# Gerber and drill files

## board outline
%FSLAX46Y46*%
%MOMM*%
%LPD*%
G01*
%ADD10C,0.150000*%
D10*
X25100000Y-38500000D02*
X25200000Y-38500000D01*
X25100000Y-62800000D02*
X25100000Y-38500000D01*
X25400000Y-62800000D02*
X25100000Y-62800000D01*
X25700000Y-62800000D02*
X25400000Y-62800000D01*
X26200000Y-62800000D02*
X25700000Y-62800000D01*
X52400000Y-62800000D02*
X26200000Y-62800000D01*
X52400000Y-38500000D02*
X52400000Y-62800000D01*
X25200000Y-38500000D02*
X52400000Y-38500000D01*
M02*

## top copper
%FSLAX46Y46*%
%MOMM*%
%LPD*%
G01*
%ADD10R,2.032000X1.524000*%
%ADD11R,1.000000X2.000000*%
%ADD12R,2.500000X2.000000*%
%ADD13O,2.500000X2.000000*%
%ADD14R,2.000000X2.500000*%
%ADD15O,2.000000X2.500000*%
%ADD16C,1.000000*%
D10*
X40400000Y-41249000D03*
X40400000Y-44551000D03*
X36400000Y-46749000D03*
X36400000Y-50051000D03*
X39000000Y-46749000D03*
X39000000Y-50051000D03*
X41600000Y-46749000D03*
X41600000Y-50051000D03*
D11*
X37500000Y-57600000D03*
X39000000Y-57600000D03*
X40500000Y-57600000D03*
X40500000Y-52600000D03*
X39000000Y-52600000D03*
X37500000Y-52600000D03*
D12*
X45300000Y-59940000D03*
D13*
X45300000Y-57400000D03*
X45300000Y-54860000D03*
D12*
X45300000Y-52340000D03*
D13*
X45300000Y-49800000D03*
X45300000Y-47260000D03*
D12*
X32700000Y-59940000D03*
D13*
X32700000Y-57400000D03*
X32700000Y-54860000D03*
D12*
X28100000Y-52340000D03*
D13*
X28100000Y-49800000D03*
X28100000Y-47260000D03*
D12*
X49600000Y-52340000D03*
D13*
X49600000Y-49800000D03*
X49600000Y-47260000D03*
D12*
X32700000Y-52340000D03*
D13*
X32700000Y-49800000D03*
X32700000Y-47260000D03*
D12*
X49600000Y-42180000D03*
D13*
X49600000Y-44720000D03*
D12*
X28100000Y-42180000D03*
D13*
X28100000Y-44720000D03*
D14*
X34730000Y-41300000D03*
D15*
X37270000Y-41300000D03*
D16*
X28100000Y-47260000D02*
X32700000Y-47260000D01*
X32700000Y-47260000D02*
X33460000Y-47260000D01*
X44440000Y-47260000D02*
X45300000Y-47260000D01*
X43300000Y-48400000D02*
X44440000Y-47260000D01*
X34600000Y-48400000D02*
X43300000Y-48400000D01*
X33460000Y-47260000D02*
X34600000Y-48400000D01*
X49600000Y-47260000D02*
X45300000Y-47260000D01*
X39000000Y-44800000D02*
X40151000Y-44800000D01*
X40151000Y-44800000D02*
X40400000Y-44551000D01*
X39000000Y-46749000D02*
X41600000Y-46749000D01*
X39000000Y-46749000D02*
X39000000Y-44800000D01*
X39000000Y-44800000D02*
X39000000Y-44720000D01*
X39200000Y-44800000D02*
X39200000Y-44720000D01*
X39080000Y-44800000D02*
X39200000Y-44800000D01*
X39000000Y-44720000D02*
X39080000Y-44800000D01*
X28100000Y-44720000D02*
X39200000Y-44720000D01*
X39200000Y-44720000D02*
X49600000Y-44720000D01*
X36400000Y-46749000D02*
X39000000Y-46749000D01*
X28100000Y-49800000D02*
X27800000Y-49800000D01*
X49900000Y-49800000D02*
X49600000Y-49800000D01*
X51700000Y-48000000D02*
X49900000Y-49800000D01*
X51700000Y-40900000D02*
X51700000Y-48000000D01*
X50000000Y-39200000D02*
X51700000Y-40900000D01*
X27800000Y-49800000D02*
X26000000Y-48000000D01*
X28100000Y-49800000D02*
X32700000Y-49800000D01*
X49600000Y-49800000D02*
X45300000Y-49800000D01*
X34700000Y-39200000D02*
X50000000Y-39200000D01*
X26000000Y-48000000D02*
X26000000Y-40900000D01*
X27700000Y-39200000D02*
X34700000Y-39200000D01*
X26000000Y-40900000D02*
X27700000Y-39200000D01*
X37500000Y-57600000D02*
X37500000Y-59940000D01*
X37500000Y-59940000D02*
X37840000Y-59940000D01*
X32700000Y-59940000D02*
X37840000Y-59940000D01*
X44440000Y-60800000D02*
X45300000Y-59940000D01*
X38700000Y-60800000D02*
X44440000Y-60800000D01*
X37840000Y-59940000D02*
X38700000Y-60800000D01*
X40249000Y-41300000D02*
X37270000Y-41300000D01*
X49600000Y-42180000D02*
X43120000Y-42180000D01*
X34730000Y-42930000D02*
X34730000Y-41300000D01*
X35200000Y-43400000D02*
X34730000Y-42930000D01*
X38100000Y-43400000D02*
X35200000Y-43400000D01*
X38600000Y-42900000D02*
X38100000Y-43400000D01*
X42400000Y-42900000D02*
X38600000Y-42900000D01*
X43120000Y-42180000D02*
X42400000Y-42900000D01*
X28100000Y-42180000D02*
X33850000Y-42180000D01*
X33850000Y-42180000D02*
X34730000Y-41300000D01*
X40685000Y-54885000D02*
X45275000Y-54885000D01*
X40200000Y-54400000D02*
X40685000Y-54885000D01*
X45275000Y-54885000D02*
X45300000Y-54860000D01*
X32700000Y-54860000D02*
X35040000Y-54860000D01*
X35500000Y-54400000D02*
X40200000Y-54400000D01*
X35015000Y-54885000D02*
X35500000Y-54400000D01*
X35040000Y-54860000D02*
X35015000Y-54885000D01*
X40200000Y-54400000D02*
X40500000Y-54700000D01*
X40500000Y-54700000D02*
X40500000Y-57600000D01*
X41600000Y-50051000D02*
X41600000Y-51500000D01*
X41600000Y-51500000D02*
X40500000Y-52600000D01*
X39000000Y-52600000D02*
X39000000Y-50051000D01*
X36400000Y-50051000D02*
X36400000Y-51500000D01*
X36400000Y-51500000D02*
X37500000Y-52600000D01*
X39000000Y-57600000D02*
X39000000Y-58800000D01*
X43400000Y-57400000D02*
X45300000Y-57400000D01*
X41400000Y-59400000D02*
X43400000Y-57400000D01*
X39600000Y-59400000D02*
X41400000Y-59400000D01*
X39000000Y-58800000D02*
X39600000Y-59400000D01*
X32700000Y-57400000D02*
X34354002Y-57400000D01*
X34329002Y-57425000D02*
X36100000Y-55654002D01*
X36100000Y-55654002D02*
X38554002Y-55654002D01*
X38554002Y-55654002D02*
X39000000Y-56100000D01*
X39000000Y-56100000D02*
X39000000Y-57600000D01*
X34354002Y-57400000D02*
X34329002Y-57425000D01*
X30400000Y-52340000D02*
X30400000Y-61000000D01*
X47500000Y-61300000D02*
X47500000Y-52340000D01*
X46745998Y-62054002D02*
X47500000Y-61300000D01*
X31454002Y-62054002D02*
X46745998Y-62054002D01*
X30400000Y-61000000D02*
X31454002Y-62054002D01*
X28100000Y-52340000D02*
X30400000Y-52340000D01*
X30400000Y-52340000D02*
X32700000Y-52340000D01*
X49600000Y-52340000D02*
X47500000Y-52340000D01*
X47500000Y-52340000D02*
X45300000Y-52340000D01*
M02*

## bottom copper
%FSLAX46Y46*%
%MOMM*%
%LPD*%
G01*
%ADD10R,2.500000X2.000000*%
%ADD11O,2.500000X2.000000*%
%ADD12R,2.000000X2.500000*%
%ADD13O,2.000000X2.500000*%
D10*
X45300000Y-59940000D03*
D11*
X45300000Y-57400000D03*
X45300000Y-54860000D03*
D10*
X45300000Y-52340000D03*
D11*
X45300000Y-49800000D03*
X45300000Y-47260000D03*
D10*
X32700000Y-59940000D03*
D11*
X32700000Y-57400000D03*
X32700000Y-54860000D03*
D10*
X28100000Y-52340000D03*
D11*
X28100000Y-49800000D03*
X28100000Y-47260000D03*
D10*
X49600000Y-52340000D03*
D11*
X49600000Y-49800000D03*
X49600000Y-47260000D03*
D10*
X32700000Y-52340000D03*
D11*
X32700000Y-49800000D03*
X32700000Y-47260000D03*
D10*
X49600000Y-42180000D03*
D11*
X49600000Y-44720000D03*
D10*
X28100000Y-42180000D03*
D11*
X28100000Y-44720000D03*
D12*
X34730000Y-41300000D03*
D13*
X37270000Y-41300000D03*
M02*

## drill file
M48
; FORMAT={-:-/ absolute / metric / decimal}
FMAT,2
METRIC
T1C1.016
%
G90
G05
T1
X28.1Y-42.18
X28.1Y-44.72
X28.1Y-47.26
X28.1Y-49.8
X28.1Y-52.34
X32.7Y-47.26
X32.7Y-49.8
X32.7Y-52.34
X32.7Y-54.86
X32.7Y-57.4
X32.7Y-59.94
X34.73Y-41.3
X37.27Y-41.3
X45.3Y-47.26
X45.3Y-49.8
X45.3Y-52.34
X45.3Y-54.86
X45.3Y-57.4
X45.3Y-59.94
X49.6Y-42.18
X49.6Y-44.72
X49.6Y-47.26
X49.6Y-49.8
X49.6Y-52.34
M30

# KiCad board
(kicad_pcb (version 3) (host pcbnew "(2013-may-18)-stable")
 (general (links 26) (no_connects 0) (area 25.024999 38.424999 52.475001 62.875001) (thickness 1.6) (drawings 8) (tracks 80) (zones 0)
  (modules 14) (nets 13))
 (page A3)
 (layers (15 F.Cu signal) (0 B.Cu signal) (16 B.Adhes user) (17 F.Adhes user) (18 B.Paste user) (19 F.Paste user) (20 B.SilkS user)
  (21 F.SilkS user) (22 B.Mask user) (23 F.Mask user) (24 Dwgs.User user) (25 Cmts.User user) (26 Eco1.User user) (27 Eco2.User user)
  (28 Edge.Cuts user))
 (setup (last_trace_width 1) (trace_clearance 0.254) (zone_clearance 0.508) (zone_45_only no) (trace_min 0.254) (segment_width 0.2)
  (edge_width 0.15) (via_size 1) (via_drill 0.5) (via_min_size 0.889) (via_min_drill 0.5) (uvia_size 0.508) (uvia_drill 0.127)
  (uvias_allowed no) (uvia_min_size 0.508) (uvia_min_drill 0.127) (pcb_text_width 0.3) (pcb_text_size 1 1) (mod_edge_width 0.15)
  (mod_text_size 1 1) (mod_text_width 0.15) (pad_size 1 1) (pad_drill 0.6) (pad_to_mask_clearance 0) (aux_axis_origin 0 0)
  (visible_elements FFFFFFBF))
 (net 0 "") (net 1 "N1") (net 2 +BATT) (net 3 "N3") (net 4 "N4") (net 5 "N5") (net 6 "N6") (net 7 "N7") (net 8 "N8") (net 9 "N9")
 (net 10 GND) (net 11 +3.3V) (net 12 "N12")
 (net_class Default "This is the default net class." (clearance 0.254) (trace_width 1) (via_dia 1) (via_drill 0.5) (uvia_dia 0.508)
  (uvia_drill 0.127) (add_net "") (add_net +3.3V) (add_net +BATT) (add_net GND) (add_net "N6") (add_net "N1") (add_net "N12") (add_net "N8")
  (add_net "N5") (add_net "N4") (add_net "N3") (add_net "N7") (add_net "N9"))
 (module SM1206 (layer F.Cu) (at 40.4 42.9 270)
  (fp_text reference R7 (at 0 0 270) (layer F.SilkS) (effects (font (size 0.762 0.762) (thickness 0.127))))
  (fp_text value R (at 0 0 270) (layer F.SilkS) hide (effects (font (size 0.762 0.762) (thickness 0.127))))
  (pad 1 smd rect (at -1.651 0 270) (size 1.524 2.032) (layers F.Cu F.Paste F.Mask) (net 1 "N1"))
  (pad 2 smd rect (at 1.651 0 270) (size 1.524 2.032) (layers F.Cu F.Paste F.Mask) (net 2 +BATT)))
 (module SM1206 (layer F.Cu) (at 36.4 48.4 270)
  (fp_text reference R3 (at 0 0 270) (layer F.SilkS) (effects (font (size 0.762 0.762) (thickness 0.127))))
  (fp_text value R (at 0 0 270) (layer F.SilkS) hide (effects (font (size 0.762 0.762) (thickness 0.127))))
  (pad 1 smd rect (at -1.651 0 270) (size 1.524 2.032) (layers F.Cu F.Paste F.Mask) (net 2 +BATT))
  (pad 2 smd rect (at 1.651 0 270) (size 1.524 2.032) (layers F.Cu F.Paste F.Mask) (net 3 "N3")))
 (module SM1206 (layer F.Cu) (at 39 48.4 270)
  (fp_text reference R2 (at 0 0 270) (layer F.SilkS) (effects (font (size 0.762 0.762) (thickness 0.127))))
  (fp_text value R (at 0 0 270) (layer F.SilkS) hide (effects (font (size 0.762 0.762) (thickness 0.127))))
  (pad 1 smd rect (at -1.651 0 270) (size 1.524 2.032) (layers F.Cu F.Paste F.Mask) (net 2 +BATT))
  (pad 2 smd rect (at 1.651 0 270) (size 1.524 2.032) (layers F.Cu F.Paste F.Mask) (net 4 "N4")))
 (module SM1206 (layer F.Cu) (at 41.6 48.4 270)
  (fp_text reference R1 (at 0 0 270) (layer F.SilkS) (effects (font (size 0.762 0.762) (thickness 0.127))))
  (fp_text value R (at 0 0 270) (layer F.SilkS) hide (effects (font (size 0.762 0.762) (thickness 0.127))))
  (pad 1 smd rect (at -1.651 0 270) (size 1.524 2.032) (layers F.Cu F.Paste F.Mask) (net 2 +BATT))
  (pad 2 smd rect (at 1.651 0 270) (size 1.524 2.032) (layers F.Cu F.Paste F.Mask) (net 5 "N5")))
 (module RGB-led (layer F.Cu) (at 39 55.1 270)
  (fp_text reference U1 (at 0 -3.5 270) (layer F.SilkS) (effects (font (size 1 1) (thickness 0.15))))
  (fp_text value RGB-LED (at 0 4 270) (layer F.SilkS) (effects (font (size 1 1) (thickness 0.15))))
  (pad 1 smd rect (at 2.5 1.5 270) (size 2 1) (layers F.Cu F.Paste F.Mask) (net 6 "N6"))
  (pad 2 smd rect (at 2.5 0 270) (size 2 1) (layers F.Cu F.Paste F.Mask) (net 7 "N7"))
  (pad 3 smd rect (at 2.5 -1.5 270) (size 2 1) (layers F.Cu F.Paste F.Mask) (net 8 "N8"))
  (pad 4 smd rect (at -2.5 -1.5 270) (size 2 1) (layers F.Cu F.Paste F.Mask) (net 5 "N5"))
  (pad 5 smd rect (at -2.5 0 270) (size 2 1) (layers F.Cu F.Paste F.Mask) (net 4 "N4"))
  (pad 6 smd rect (at -2.5 1.5 270) (size 2 1) (layers F.Cu F.Paste F.Mask) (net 3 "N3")))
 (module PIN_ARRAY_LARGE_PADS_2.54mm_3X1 (layer F.Cu) (at 45.3 57.4 90)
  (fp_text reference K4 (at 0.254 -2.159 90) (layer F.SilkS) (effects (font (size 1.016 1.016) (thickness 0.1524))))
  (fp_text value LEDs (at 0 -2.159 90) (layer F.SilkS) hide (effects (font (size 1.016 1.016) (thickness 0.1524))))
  (pad 1 thru_hole rect (at -2.54 0 90) (size 2 2.5) (drill 1.016) (layers *.Cu *.Mask F.SilkS) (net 6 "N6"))
  (pad 2 thru_hole oval (at 0 0 90) (size 2 2.5) (drill 1.016) (layers *.Cu *.Mask F.SilkS) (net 7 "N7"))
  (pad 3 thru_hole oval (at 2.54 0 90) (size 2 2.5) (drill 1.016) (layers *.Cu *.Mask F.SilkS) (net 8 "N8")))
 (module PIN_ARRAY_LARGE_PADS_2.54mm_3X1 (layer F.Cu) (at 45.3 49.8 90)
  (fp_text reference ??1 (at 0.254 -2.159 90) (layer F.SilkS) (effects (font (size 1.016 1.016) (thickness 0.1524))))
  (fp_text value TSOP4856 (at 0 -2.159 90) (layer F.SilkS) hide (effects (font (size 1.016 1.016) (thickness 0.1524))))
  (pad 1 thru_hole rect (at -2.54 0 90) (size 2 2.5) (drill 1.016) (layers *.Cu *.Mask F.SilkS) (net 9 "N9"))
  (pad 2 thru_hole oval (at 0 0 90) (size 2 2.5) (drill 1.016) (layers *.Cu *.Mask F.SilkS) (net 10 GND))
  (pad 3 thru_hole oval (at 2.54 0 90) (size 2 2.5) (drill 1.016) (layers *.Cu *.Mask F.SilkS) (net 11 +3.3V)))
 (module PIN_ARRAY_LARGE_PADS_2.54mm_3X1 (layer F.Cu) (at 32.7 57.4 90)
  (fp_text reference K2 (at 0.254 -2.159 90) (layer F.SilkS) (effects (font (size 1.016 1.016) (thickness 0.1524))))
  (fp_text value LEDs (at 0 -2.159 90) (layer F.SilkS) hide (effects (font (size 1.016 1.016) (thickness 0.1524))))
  (pad 1 thru_hole rect (at -2.54 0 90) (size 2 2.5) (drill 1.016) (layers *.Cu *.Mask F.SilkS) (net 6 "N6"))
  (pad 2 thru_hole oval (at 0 0 90) (size 2 2.5) (drill 1.016) (layers *.Cu *.Mask F.SilkS) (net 7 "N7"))
  (pad 3 thru_hole oval (at 2.54 0 90) (size 2 2.5) (drill 1.016) (layers *.Cu *.Mask F.SilkS) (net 8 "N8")))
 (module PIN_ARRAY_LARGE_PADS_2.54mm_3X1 (layer F.Cu) (at 28.1 49.8 90)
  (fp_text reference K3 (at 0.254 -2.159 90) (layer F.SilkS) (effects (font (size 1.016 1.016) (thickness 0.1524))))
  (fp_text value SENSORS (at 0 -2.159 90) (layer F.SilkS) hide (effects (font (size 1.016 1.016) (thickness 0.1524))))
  (pad 1 thru_hole rect (at -2.54 0 90) (size 2 2.5) (drill 1.016) (layers *.Cu *.Mask F.SilkS) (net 9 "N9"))
  (pad 2 thru_hole oval (at 0 0 90) (size 2 2.5) (drill 1.016) (layers *.Cu *.Mask F.SilkS) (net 10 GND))
  (pad 3 thru_hole oval (at 2.54 0 90) (size 2 2.5) (drill 1.016) (layers *.Cu *.Mask F.SilkS) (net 11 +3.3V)))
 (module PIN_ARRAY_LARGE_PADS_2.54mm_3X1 (layer F.Cu) (at 49.6 49.8 90)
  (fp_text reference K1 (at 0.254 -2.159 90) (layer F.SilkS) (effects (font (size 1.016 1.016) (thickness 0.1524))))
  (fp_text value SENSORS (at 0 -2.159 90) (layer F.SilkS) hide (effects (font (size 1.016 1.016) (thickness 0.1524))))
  (pad 1 thru_hole rect (at -2.54 0 90) (size 2 2.5) (drill 1.016) (layers *.Cu *.Mask F.SilkS) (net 9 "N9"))
  (pad 2 thru_hole oval (at 0 0 90) (size 2 2.5) (drill 1.016) (layers *.Cu *.Mask F.SilkS) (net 10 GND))
  (pad 3 thru_hole oval (at 2.54 0 90) (size 2 2.5) (drill 1.016) (layers *.Cu *.Mask F.SilkS) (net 11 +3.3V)))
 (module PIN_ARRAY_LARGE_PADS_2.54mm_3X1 (layer F.Cu) (at 32.7 49.8 90)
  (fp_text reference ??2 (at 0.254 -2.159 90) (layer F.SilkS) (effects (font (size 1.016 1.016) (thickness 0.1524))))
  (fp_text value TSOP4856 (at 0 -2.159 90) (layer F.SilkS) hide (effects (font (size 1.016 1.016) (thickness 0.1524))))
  (pad 1 thru_hole rect (at -2.54 0 90) (size 2 2.5) (drill 1.016) (layers *.Cu *.Mask F.SilkS) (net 9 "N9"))
  (pad 2 thru_hole oval (at 0 0 90) (size 2 2.5) (drill 1.016) (layers *.Cu *.Mask F.SilkS) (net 10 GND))
  (pad 3 thru_hole oval (at 2.54 0 90) (size 2 2.5) (drill 1.016) (layers *.Cu *.Mask F.SilkS) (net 11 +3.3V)))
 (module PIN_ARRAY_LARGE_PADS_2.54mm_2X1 (layer F.Cu) (at 49.6 43.45 270)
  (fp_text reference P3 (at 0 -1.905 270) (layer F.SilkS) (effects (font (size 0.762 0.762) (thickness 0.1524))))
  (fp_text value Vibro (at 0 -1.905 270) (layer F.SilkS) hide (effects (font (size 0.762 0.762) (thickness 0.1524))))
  (pad 1 thru_hole rect (at -1.27 0 270) (size 2 2.5) (drill 1.016) (layers *.Cu *.Mask F.SilkS) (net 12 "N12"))
  (pad 2 thru_hole oval (at 1.27 0 270) (size 2 2.5) (drill 1.016) (layers *.Cu *.Mask F.SilkS) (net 2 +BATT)))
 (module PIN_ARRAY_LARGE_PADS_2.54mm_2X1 (layer F.Cu) (at 28.1 43.45 270)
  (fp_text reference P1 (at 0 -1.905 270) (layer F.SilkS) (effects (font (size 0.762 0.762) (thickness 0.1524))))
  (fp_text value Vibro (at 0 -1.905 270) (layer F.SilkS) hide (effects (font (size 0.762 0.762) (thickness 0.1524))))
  (pad 1 thru_hole rect (at -1.27 0 270) (size 2 2.5) (drill 1.016) (layers *.Cu *.Mask F.SilkS) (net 12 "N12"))
  (pad 2 thru_hole oval (at 1.27 0 270) (size 2 2.5) (drill 1.016) (layers *.Cu *.Mask F.SilkS) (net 2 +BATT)))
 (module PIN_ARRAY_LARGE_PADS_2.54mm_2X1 (layer F.Cu) (at 36 41.3)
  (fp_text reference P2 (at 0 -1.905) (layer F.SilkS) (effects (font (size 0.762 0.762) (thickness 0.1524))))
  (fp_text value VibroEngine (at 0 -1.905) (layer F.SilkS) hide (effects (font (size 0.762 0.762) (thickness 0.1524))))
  (pad 1 thru_hole rect (at -1.27 0) (size 2 2.5) (drill 1.016) (layers *.Cu *.Mask F.SilkS) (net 12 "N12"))
  (pad 2 thru_hole oval (at 1.27 0) (size 2 2.5) (drill 1.016) (layers *.Cu *.Mask F.SilkS) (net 1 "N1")))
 (gr_line (start 25.1 38.5) (end 25.2 38.5) (angle 90) (layer Edge.Cuts) (width 0.15))
 (gr_line (start 25.1 62.8) (end 25.1 38.5) (angle 90) (layer Edge.Cuts) (width 0.15))
 (gr_line (start 25.4 62.8) (end 25.1 62.8) (angle 90) (layer Edge.Cuts) (width 0.15))
 (gr_line (start 25.7 62.8) (end 25.4 62.8) (angle 90) (layer Edge.Cuts) (width 0.15))
 (gr_line (start 26.2 62.8) (end 25.7 62.8) (angle 90) (layer Edge.Cuts) (width 0.15))
 (gr_line (start 52.4 62.8) (end 26.2 62.8) (angle 90) (layer Edge.Cuts) (width 0.15))
 (gr_line (start 52.4 38.5) (end 52.4 62.8) (angle 90) (layer Edge.Cuts) (width 0.15))
 (gr_line (start 25.2 38.5) (end 52.4 38.5) (angle 90) (layer Edge.Cuts) (width 0.15))
 (segment (start 28.1 47.26) (end 32.7 47.26) (width 1) (layer F.Cu) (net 11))
 (segment (start 32.7 47.26) (end 33.46 47.26) (width 1) (layer F.Cu) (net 11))
 (segment (start 44.44 47.26) (end 45.3 47.26) (width 1) (layer F.Cu) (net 11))
 (segment (start 43.3 48.4) (end 44.44 47.26) (width 1) (layer F.Cu) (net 11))
 (segment (start 34.6 48.4) (end 43.3 48.4) (width 1) (layer F.Cu) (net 11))
 (segment (start 33.46 47.26) (end 34.6 48.4) (width 1) (layer F.Cu) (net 11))
 (segment (start 49.6 47.26) (end 45.3 47.26) (width 1) (layer F.Cu) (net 11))
 (segment (start 39 44.8) (end 40.151 44.8) (width 1) (layer F.Cu) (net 2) (status 800000))
 (segment (start 40.151 44.8) (end 40.4 44.551) (width 1) (layer F.Cu) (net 2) (status C00000))
 (segment (start 39 46.749) (end 41.6 46.749) (width 1) (layer F.Cu) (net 2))
 (segment (start 39 46.749) (end 39 44.8) (width 1) (layer F.Cu) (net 2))
 (segment (start 39 44.8) (end 39 44.72) (width 1) (layer F.Cu) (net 2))
 (segment (start 39.2 44.8) (end 39.2 44.72) (width 1) (layer F.Cu) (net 2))
 (segment (start 39.08 44.8) (end 39.2 44.8) (width 1) (layer F.Cu) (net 2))
 (segment (start 39 44.72) (end 39.08 44.8) (width 1) (layer F.Cu) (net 2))
 (segment (start 28.1 44.72) (end 39.2 44.72) (width 1) (layer F.Cu) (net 2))
 (segment (start 39.2 44.72) (end 49.6 44.72) (width 1) (layer F.Cu) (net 2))
 (segment (start 36.4 46.749) (end 39 46.749) (width 1) (layer F.Cu) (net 2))
 (segment (start 28.1 49.8) (end 27.8 49.8) (width 1) (layer F.Cu) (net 10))
 (segment (start 49.9 49.8) (end 49.6 49.8) (width 1) (layer F.Cu) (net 10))
 (segment (start 51.7 48) (end 49.9 49.8) (width 1) (layer F.Cu) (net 10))
 (segment (start 51.7 40.9) (end 51.7 48) (width 1) (layer F.Cu) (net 10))
 (segment (start 50 39.2) (end 51.7 40.9) (width 1) (layer F.Cu) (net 10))
 (segment (start 27.8 49.8) (end 26 48) (width 1) (layer F.Cu) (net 10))
 (segment (start 28.1 49.8) (end 32.7 49.8) (width 1) (layer F.Cu) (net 10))
 (segment (start 49.6 49.8) (end 45.3 49.8) (width 1) (layer F.Cu) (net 10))
 (segment (start 34.7 39.2) (end 50 39.2) (width 1) (layer F.Cu) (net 10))
 (segment (start 26 48) (end 26 40.9) (width 1) (layer F.Cu) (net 10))
 (segment (start 27.7 39.2) (end 34.7 39.2) (width 1) (layer F.Cu) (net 10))
 (segment (start 26 40.9) (end 27.7 39.2) (width 1) (layer F.Cu) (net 10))
 (segment (start 37.5 57.6) (end 37.5 59.94) (width 1) (layer F.Cu) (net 6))
 (segment (start 37.5 59.94) (end 37.84 59.94) (width 1) (layer F.Cu) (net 6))
 (segment (start 32.7 59.94) (end 37.84 59.94) (width 1) (layer F.Cu) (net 6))
 (segment (start 44.44 60.8) (end 45.3 59.94) (width 1) (layer F.Cu) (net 6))
 (segment (start 38.7 60.8) (end 44.44 60.8) (width 1) (layer F.Cu) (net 6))
 (segment (start 37.84 59.94) (end 38.7 60.8) (width 1) (layer F.Cu) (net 6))
 (segment (start 40.249 41.3) (end 37.27 41.3) (width 1) (layer F.Cu) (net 1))
 (segment (start 49.6 42.18) (end 43.12 42.18) (width 1) (layer F.Cu) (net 12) (status 400000))
 (segment (start 34.73 42.93) (end 34.73 41.3) (width 1) (layer F.Cu) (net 12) (status 800000))
 (segment (start 35.2 43.4) (end 34.73 42.93) (width 1) (layer F.Cu) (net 12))
 (segment (start 38.1 43.4) (end 35.2 43.4) (width 1) (layer F.Cu) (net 12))
 (segment (start 38.6 42.9) (end 38.1 43.4) (width 1) (layer F.Cu) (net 12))
 (segment (start 42.4 42.9) (end 38.6 42.9) (width 1) (layer F.Cu) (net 12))
 (segment (start 43.12 42.18) (end 42.4 42.9) (width 1) (layer F.Cu) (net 12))
 (segment (start 28.1 42.18) (end 33.85 42.18) (width 1) (layer F.Cu) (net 12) (status C00000))
 (segment (start 33.85 42.18) (end 34.73 41.3) (width 1) (layer F.Cu) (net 12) (status C00000))
 (segment (start 40.685 54.885) (end 45.275 54.885) (width 1) (layer F.Cu) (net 8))
 (segment (start 40.2 54.4) (end 40.685 54.885) (width 1) (layer F.Cu) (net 8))
 (segment (start 45.275 54.885) (end 45.3 54.86) (width 1) (layer F.Cu) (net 8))
 (segment (start 32.7 54.86) (end 35.04 54.86) (width 1) (layer F.Cu) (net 8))
 (segment (start 35.5 54.4) (end 40.2 54.4) (width 1) (layer F.Cu) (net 8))
 (segment (start 35.015 54.885) (end 35.5 54.4) (width 1) (layer F.Cu) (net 8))
 (segment (start 35.04 54.86) (end 35.015 54.885) (width 1) (layer F.Cu) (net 8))
 (segment (start 40.2 54.4) (end 40.5 54.7) (width 1) (layer F.Cu) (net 8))
 (segment (start 40.5 54.7) (end 40.5 57.6) (width 1) (layer F.Cu) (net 8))
 (segment (start 41.6 50.051) (end 41.6 51.5) (width 1) (layer F.Cu) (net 5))
 (segment (start 41.6 51.5) (end 40.5 52.6) (width 1) (layer F.Cu) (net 5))
 (segment (start 39 52.6) (end 39 50.051) (width 1) (layer F.Cu) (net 4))
 (segment (start 36.4 50.051) (end 36.4 51.5) (width 1) (layer F.Cu) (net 3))
 (segment (start 36.4 51.5) (end 37.5 52.6) (width 1) (layer F.Cu) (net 3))
 (segment (start 39 57.6) (end 39 58.8) (width 1) (layer F.Cu) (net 7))
 (segment (start 43.4 57.4) (end 45.3 57.4) (width 1) (layer F.Cu) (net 7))
 (segment (start 41.4 59.4) (end 43.4 57.4) (width 1) (layer F.Cu) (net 7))
 (segment (start 39.6 59.4) (end 41.4 59.4) (width 1) (layer F.Cu) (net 7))
 (segment (start 39 58.8) (end 39.6 59.4) (width 1) (layer F.Cu) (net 7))
 (segment (start 32.7 57.4) (end 34.354002 57.4) (width 1) (layer F.Cu) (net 7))
 (segment (start 34.329002 57.425) (end 36.1 55.654002) (width 1) (layer F.Cu) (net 7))
 (segment (start 36.1 55.654002) (end 38.554002 55.654002) (width 1) (layer F.Cu) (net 7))
 (segment (start 38.554002 55.654002) (end 39 56.1) (width 1) (layer F.Cu) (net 7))
 (segment (start 39 56.1) (end 39 57.6) (width 1) (layer F.Cu) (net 7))
 (segment (start 34.354002 57.4) (end 34.329002 57.425) (width 1) (layer F.Cu) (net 7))
 (segment (start 30.4 52.34) (end 30.4 61) (width 1) (layer F.Cu) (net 9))
 (segment (start 47.5 61.3) (end 47.5 52.34) (width 1) (layer F.Cu) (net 9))
 (segment (start 46.745998 62.054002) (end 47.5 61.3) (width 1) (layer F.Cu) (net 9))
 (segment (start 31.454002 62.054002) (end 46.745998 62.054002) (width 1) (layer F.Cu) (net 9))
 (segment (start 30.4 61) (end 31.454002 62.054002) (width 1) (layer F.Cu) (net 9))
 (segment (start 28.1 52.34) (end 30.4 52.34) (width 1) (layer F.Cu) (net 9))
 (segment (start 30.4 52.34) (end 32.7 52.34) (width 1) (layer F.Cu) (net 9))
 (segment (start 49.6 52.34) (end 47.5 52.34) (width 1) (layer F.Cu) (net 9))
 (segment (start 47.5 52.34) (end 45.3 52.34) (width 1) (layer F.Cu) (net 9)))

